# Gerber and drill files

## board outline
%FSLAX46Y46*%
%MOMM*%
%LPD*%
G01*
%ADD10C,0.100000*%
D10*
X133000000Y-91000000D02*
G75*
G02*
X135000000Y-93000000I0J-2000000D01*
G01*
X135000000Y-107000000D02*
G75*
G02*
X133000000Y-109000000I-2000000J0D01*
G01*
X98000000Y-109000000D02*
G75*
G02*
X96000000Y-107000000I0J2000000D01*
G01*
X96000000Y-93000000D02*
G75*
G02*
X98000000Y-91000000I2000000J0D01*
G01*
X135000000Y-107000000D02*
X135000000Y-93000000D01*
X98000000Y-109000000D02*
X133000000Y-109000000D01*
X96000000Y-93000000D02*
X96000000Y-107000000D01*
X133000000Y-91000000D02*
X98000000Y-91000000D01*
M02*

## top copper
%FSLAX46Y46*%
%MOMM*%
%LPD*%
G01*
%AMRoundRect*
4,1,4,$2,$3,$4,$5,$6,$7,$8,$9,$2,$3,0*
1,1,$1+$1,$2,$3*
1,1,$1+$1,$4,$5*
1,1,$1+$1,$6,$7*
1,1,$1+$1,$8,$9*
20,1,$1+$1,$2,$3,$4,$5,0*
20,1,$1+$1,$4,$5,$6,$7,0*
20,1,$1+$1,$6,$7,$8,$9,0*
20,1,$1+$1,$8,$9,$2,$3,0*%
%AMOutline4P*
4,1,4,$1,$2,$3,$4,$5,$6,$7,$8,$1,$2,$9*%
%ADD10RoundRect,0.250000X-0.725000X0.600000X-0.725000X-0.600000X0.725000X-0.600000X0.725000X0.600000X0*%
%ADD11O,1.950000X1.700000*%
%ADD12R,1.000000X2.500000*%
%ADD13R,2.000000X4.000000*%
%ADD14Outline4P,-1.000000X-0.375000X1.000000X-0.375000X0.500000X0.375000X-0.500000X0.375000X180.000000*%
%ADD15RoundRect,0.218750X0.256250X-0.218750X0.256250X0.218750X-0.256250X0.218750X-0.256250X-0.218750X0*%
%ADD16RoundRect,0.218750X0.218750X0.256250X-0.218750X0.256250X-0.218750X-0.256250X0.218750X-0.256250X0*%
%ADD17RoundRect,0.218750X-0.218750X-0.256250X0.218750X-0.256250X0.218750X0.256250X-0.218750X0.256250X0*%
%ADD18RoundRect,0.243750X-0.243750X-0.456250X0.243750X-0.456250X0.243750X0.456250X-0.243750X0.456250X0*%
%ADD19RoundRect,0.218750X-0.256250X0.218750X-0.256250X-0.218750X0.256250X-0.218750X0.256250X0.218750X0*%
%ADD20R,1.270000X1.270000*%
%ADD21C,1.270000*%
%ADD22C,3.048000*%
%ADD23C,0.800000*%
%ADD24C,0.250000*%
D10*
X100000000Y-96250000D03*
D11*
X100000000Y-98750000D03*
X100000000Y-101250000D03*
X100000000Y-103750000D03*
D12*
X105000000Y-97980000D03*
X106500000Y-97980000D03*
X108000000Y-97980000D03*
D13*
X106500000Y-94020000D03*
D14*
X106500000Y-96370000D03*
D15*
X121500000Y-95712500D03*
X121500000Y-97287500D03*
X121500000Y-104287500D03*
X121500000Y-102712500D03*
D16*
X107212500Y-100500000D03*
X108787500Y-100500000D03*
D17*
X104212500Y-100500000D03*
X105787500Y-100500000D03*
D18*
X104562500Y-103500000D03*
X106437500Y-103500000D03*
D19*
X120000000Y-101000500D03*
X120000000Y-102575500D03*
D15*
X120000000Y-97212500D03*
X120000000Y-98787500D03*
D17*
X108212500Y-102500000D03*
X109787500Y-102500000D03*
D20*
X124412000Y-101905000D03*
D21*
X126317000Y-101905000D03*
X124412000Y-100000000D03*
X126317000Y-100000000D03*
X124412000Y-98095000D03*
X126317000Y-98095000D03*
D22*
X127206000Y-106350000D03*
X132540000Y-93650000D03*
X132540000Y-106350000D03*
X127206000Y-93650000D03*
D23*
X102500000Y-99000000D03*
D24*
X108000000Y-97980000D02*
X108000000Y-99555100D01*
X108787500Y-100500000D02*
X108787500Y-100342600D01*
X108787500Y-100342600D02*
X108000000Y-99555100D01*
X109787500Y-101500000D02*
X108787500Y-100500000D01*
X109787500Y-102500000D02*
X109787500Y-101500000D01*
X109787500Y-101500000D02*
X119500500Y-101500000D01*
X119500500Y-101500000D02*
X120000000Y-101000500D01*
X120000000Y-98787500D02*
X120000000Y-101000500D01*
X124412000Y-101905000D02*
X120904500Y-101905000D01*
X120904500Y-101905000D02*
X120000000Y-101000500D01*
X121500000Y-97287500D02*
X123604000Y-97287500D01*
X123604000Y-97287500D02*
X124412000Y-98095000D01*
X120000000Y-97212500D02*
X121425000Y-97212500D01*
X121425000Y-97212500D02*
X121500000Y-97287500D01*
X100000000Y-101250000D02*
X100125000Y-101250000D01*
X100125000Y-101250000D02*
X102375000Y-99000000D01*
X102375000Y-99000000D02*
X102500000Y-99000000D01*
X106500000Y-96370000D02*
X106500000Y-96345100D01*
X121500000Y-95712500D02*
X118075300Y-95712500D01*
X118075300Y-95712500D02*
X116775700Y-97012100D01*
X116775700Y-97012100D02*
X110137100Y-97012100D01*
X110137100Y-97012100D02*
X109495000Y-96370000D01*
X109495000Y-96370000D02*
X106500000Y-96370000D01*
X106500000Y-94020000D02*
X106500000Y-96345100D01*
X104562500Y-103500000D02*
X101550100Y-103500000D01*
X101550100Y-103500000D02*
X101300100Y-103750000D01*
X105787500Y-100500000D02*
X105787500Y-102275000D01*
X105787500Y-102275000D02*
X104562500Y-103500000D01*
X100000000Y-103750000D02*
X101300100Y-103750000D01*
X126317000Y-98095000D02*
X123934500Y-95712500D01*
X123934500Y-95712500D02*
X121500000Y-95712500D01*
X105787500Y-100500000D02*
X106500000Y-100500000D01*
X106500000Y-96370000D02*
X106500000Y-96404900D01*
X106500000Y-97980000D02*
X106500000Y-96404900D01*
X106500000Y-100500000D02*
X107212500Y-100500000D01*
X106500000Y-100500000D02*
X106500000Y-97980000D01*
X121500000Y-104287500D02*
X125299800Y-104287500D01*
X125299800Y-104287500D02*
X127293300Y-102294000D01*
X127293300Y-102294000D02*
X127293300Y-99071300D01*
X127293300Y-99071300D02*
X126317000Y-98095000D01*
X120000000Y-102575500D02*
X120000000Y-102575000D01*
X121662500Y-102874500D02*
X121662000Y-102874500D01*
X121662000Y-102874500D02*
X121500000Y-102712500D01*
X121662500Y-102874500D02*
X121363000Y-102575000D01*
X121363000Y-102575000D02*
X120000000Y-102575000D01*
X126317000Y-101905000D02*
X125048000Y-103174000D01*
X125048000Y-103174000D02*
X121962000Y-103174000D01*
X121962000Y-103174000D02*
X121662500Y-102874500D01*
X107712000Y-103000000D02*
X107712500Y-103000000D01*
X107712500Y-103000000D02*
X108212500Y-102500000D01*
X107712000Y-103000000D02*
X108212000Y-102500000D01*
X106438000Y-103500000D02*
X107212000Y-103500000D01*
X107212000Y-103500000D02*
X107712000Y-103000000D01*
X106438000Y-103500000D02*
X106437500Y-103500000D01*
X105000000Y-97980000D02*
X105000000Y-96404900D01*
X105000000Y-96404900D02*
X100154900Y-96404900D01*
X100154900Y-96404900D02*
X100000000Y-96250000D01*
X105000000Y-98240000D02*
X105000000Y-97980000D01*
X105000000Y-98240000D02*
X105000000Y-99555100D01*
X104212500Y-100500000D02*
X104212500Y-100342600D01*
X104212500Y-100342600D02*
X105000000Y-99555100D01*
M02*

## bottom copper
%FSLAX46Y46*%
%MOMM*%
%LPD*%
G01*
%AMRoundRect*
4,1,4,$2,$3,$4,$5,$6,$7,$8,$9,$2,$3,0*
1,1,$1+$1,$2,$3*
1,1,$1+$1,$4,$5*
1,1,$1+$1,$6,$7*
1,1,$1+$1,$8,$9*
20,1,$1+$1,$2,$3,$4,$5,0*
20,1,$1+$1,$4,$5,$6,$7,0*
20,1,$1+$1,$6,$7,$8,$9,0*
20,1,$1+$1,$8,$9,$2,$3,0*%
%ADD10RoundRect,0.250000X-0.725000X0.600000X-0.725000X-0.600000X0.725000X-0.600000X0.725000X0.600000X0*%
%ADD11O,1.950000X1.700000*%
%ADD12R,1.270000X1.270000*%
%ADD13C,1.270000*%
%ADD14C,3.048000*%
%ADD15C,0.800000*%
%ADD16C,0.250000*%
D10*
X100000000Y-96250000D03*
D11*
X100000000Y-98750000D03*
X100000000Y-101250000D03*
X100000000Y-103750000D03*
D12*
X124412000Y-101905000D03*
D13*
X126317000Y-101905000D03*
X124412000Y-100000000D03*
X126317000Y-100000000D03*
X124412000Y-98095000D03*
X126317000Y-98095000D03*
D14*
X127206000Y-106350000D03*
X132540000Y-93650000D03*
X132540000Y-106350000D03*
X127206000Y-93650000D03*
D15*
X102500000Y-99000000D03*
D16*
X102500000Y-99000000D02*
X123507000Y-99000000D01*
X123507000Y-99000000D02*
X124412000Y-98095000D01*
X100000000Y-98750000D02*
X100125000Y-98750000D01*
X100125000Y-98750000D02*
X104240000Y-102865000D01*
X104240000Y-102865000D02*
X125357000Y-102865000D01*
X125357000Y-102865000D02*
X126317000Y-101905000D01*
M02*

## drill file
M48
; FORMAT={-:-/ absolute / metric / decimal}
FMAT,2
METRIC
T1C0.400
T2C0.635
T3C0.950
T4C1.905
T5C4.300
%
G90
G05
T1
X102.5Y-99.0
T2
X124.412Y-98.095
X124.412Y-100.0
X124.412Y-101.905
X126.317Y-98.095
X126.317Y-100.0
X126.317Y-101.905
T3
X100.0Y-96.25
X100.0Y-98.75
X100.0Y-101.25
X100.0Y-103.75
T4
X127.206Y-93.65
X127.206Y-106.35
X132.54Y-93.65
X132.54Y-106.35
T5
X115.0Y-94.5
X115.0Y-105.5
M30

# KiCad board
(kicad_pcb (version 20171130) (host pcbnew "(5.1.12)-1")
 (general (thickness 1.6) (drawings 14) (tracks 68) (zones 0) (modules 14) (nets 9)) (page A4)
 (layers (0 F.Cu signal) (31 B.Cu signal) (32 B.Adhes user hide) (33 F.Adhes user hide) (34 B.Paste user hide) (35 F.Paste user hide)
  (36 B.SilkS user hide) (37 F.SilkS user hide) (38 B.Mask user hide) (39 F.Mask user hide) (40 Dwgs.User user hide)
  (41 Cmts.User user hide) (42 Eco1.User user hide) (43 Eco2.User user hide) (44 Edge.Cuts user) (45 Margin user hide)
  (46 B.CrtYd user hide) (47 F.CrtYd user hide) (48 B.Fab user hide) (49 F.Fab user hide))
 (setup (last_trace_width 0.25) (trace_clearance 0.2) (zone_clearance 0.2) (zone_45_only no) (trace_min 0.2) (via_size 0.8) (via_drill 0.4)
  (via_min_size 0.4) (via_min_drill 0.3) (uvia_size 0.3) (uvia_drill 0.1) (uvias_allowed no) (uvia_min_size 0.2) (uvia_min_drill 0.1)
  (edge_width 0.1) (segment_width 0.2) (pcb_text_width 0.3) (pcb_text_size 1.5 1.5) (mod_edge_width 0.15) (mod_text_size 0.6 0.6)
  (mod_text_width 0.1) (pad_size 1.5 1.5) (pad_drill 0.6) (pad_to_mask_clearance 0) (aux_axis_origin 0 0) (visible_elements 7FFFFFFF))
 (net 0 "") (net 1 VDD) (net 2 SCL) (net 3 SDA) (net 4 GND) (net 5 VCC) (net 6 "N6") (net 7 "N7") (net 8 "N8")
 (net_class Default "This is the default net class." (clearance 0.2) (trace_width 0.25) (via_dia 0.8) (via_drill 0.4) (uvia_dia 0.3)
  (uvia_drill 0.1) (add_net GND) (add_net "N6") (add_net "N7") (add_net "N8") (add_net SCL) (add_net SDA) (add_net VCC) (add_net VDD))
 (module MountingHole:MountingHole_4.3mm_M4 (layer F.Cu) (at 115 105.5)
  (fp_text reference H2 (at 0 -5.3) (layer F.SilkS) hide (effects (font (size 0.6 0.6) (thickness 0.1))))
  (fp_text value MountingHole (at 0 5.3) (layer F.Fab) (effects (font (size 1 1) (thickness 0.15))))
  (pad 1 np_thru_hole circle (at 0 0) (size 4.3 4.3) (drill 4.3) (layers *.Cu *.Mask)))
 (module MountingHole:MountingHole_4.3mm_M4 (layer F.Cu) (at 115 94.5)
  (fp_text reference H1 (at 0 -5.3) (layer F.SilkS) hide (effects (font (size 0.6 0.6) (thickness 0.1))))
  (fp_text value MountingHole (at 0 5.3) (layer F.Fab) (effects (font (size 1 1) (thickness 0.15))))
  (pad 1 np_thru_hole circle (at 0 0) (size 4.3 4.3) (drill 4.3) (layers *.Cu *.Mask)))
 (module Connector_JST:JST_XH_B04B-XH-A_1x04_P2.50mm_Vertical (layer F.Cu) (at 100 96.25 270)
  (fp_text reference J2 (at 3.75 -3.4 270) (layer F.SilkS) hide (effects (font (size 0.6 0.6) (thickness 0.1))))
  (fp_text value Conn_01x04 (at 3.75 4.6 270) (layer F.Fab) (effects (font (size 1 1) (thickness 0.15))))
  (pad 1 thru_hole roundrect (at 0 0 270) (size 1.7 1.95) (drill 0.95) (layers *.Cu *.Mask) (roundrect_rratio 0.147059) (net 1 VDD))
  (pad 2 thru_hole oval (at 2.5 0 270) (size 1.7 1.95) (drill 0.95) (layers *.Cu *.Mask) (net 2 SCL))
  (pad 3 thru_hole oval (at 5 0 270) (size 1.7 1.95) (drill 0.95) (layers *.Cu *.Mask) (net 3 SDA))
  (pad 4 thru_hole oval (at 7.5 0 270) (size 1.7 1.95) (drill 0.95) (layers *.Cu *.Mask) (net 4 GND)))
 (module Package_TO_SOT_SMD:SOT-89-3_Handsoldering (layer F.Cu) (at 106.5 96 90)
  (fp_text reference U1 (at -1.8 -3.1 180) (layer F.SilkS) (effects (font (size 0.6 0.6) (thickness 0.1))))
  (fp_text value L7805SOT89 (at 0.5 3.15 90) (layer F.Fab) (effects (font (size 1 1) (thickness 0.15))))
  (pad 1 smd rect (at -1.98 -1.5) (size 1 2.5) (layers F.Cu F.Paste F.Mask) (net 1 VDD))
  (pad 2 smd rect (at -1.98 0) (size 1 2.5) (layers F.Cu F.Paste F.Mask) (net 4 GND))
  (pad 3 smd rect (at -1.98 1.5) (size 1 2.5) (layers F.Cu F.Paste F.Mask) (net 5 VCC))
  (pad 2 smd rect (at 1.98 0) (size 2 4) (layers F.Cu F.Paste F.Mask) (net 4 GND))
  (pad 2 smd trapezoid (at -0.37 0 180) (size 1.5 0.75) (rect_delta 0 0.5) (layers F.Cu F.Paste F.Mask) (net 4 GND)))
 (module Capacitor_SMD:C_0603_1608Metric (layer F.Cu) (at 121.5 96.5 90)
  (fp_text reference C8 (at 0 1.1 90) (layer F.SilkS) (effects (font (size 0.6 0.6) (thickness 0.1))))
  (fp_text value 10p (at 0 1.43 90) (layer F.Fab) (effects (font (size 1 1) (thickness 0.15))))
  (pad 2 smd roundrect (at 0.7875 0 90) (size 0.875 0.95) (layers F.Cu F.Paste F.Mask) (roundrect_rratio 0.25) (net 4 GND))
  (pad 1 smd roundrect (at -0.7875 0 90) (size 0.875 0.95) (layers F.Cu F.Paste F.Mask) (roundrect_rratio 0.25) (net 3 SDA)))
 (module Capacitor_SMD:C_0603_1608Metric (layer F.Cu) (at 121.5 103.5 90)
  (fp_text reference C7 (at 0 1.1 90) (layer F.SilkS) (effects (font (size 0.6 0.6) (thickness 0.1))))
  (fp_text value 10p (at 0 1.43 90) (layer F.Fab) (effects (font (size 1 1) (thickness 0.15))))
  (pad 1 smd roundrect (at -0.7875 0 90) (size 0.875 0.95) (layers F.Cu F.Paste F.Mask) (roundrect_rratio 0.25) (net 4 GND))
  (pad 2 smd roundrect (at 0.7875 0 90) (size 0.875 0.95) (layers F.Cu F.Paste F.Mask) (roundrect_rratio 0.25) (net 2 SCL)))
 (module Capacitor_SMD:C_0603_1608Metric (layer F.Cu) (at 108 100.5 180)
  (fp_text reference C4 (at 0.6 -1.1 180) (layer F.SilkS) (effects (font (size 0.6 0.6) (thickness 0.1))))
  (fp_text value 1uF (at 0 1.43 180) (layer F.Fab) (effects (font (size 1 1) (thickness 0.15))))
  (pad 2 smd roundrect (at 0.7875 0 180) (size 0.875 0.95) (layers F.Cu F.Paste F.Mask) (roundrect_rratio 0.25) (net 4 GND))
  (pad 1 smd roundrect (at -0.7875 0 180) (size 0.875 0.95) (layers F.Cu F.Paste F.Mask) (roundrect_rratio 0.25) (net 5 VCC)))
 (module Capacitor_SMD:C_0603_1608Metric (layer F.Cu) (at 105 100.5)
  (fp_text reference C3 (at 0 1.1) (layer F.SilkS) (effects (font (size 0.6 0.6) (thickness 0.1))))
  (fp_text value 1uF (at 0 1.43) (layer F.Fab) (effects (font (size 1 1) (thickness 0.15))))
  (pad 1 smd roundrect (at -0.7875 0) (size 0.875 0.95) (layers F.Cu F.Paste F.Mask) (roundrect_rratio 0.25) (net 1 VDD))
  (pad 2 smd roundrect (at 0.7875 0) (size 0.875 0.95) (layers F.Cu F.Paste F.Mask) (roundrect_rratio 0.25) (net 4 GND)))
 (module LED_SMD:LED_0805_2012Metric (layer F.Cu) (at 105.5 103.5)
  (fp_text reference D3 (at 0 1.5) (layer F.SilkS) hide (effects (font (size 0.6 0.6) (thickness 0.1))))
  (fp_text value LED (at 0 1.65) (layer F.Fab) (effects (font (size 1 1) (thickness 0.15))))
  (pad 1 smd roundrect (at -0.9375 0) (size 0.975 1.4) (layers F.Cu F.Paste F.Mask) (roundrect_rratio 0.25) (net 4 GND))
  (pad 2 smd roundrect (at 0.9375 0) (size 0.975 1.4) (layers F.Cu F.Paste F.Mask) (roundrect_rratio 0.25) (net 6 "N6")))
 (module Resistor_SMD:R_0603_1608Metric (layer F.Cu) (at 120 101.788 270)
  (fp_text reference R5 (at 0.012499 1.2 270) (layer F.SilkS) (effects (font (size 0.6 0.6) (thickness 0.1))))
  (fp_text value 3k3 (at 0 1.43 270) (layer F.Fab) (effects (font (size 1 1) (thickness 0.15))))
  (pad 1 smd roundrect (at -0.7875 0 270) (size 0.875 0.95) (layers F.Cu F.Paste F.Mask) (roundrect_rratio 0.25) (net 5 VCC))
  (pad 2 smd roundrect (at 0.7875 0 270) (size 0.875 0.95) (layers F.Cu F.Paste F.Mask) (roundrect_rratio 0.25) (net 2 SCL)))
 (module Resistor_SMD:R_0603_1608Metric (layer F.Cu) (at 120 98 90)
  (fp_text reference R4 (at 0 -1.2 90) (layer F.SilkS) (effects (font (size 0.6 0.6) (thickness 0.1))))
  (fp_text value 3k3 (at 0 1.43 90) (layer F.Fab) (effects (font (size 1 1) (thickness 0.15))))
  (pad 2 smd roundrect (at 0.7875 0 90) (size 0.875 0.95) (layers F.Cu F.Paste F.Mask) (roundrect_rratio 0.25) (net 3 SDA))
  (pad 1 smd roundrect (at -0.7875 0 90) (size 0.875 0.95) (layers F.Cu F.Paste F.Mask) (roundrect_rratio 0.25) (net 5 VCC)))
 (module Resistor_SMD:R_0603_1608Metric (layer F.Cu) (at 109 102.5)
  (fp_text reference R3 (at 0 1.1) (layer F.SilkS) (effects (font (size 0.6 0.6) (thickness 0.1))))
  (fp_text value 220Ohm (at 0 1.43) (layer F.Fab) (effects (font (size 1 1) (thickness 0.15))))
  (pad 1 smd roundrect (at -0.7875 0) (size 0.875 0.95) (layers F.Cu F.Paste F.Mask) (roundrect_rratio 0.25) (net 6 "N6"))
  (pad 2 smd roundrect (at 0.7875 0) (size 0.875 0.95) (layers F.Cu F.Paste F.Mask) (roundrect_rratio 0.25) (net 5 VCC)))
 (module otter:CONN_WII (layer F.Cu) (at 130 100 270)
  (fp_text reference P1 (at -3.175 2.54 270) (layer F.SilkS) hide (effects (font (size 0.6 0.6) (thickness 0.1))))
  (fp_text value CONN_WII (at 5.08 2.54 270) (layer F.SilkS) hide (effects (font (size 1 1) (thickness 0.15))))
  (pad 1 thru_hole rect (at 1.905 5.588 270) (size 1.27 1.27) (drill 0.635) (layers *.Cu *.Mask F.SilkS) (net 5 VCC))
  (pad 2 thru_hole circle (at 1.905 3.683 270) (size 1.27 1.27) (drill 0.635) (layers *.Cu *.Mask F.SilkS) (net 2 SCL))
  (pad 3 thru_hole circle (at 0 5.588 270) (size 1.27 1.27) (drill 0.635) (layers *.Cu *.Mask F.SilkS) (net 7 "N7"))
  (pad 4 thru_hole circle (at 0 3.683 270) (size 1.27 1.27) (drill 0.635) (layers *.Cu *.Mask F.SilkS) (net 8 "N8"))
  (pad 5 thru_hole circle (at -1.905 5.588 270) (size 1.27 1.27) (drill 0.635) (layers *.Cu *.Mask F.SilkS) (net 3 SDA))
  (pad 6 thru_hole circle (at -1.905 3.683 270) (size 1.27 1.27) (drill 0.635) (layers *.Cu *.Mask F.SilkS) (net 4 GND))
  (pad "" thru_hole circle (at 6.35 2.794 270) (size 3.048 3.048) (drill 1.905) (layers *.Cu *.Mask F.SilkS))
  (pad "" thru_hole circle (at -6.35 -2.54 270) (size 3.048 3.048) (drill 1.905) (layers *.Cu *.Mask F.SilkS))
  (pad "" thru_hole circle (at 6.35 -2.54 270) (size 3.048 3.048) (drill 1.905) (layers *.Cu *.Mask F.SilkS))
  (pad "" thru_hole circle (at -6.35 2.794 270) (size 3.048 3.048) (drill 1.905) (layers *.Cu *.Mask F.SilkS)))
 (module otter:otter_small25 (layer B.Cu) (at 107 100 180)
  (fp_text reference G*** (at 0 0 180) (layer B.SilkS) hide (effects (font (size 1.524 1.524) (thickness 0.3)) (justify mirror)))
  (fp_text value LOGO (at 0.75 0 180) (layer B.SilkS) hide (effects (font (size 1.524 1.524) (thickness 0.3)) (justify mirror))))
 (gr_arc (start 133 93) (end 135 93) (angle -90) (layer Edge.Cuts) (width 0.1))
 (gr_arc (start 133 107) (end 133 109) (angle -90) (layer Edge.Cuts) (width 0.1))
 (gr_arc (start 98 107) (end 96 107) (angle -90) (layer Edge.Cuts) (width 0.1))
 (gr_arc (start 98 93) (end 98 91) (angle -90) (layer Edge.Cuts) (width 0.1))
 (gr_line (start 135 107) (end 135 93) (layer Edge.Cuts) (width 0.1))
 (gr_line (start 98 109) (end 133 109) (layer Edge.Cuts) (width 0.1))
 (gr_line (start 96 93) (end 96 107) (layer Edge.Cuts) (width 0.1))
 (gr_line (start 133 91) (end 98 91) (layer Edge.Cuts) (width 0.1))
 (segment (start 108 97.98) (end 108 99.5551) (width 0.25) (layer F.Cu) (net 5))
 (segment (start 108.7875 100.5) (end 108.7875 100.3426) (width 0.25) (layer F.Cu) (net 5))
 (segment (start 108.7875 100.3426) (end 108 99.5551) (width 0.25) (layer F.Cu) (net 5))
 (segment (start 109.7875 101.5) (end 108.7875 100.5) (width 0.25) (layer F.Cu) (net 5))
 (segment (start 109.7875 102.5) (end 109.7875 101.5) (width 0.25) (layer F.Cu) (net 5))
 (segment (start 109.7875 101.5) (end 119.5005 101.5) (width 0.25) (layer F.Cu) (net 5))
 (segment (start 119.5005 101.5) (end 120 101.0005) (width 0.25) (layer F.Cu) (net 5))
 (segment (start 120 98.7875) (end 120 101.0005) (width 0.25) (layer F.Cu) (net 5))
 (segment (start 124.412 101.905) (end 120.9045 101.905) (width 0.25) (layer F.Cu) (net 5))
 (segment (start 120.9045 101.905) (end 120 101.0005) (width 0.25) (layer F.Cu) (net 5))
 (segment (start 121.5 97.2875) (end 123.604 97.2875) (width 0.25) (layer F.Cu) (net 3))
 (segment (start 123.604 97.2875) (end 124.412 98.095) (width 0.25) (layer F.Cu) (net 3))
 (segment (start 120 97.2125) (end 121.425 97.2125) (width 0.25) (layer F.Cu) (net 3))
 (segment (start 121.425 97.2125) (end 121.5 97.2875) (width 0.25) (layer F.Cu) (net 3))
 (segment (start 102.5 99) (end 123.507 99) (width 0.25) (layer B.Cu) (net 3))
 (segment (start 123.507 99) (end 124.412 98.095) (width 0.25) (layer B.Cu) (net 3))
 (segment (start 100 101.25) (end 100.125 101.25) (width 0.25) (layer F.Cu) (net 3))
 (segment (start 100.125 101.25) (end 102.375 99) (width 0.25) (layer F.Cu) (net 3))
 (segment (start 102.375 99) (end 102.5 99) (width 0.25) (layer F.Cu) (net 3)) (via (at 102.5 99) (size 0.8) (layers F.Cu B.Cu) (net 3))
 (segment (start 106.5 96.37) (end 106.5 96.3451) (width 0.25) (layer F.Cu) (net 4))
 (segment (start 121.5 95.7125) (end 118.0753 95.7125) (width 0.25) (layer F.Cu) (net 4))
 (segment (start 118.0753 95.7125) (end 116.7757 97.0121) (width 0.25) (layer F.Cu) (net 4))
 (segment (start 116.7757 97.0121) (end 110.1371 97.0121) (width 0.25) (layer F.Cu) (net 4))
 (segment (start 110.1371 97.0121) (end 109.495 96.37) (width 0.25) (layer F.Cu) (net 4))
 (segment (start 109.495 96.37) (end 106.5 96.37) (width 0.25) (layer F.Cu) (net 4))
 (segment (start 106.5 94.02) (end 106.5 96.3451) (width 0.25) (layer F.Cu) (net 4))
 (segment (start 104.5625 103.5) (end 101.5501 103.5) (width 0.25) (layer F.Cu) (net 4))
 (segment (start 101.5501 103.5) (end 101.3001 103.75) (width 0.25) (layer F.Cu) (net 4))
 (segment (start 105.7875 100.5) (end 105.7875 102.275) (width 0.25) (layer F.Cu) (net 4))
 (segment (start 105.7875 102.275) (end 104.5625 103.5) (width 0.25) (layer F.Cu) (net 4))
 (segment (start 100 103.75) (end 101.3001 103.75) (width 0.25) (layer F.Cu) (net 4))
 (segment (start 126.317 98.095) (end 123.9345 95.7125) (width 0.25) (layer F.Cu) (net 4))
 (segment (start 123.9345 95.7125) (end 121.5 95.7125) (width 0.25) (layer F.Cu) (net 4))
 (segment (start 105.7875 100.5) (end 106.5 100.5) (width 0.25) (layer F.Cu) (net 4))
 (segment (start 106.5 96.37) (end 106.5 96.4049) (width 0.25) (layer F.Cu) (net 4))
 (segment (start 106.5 97.98) (end 106.5 96.4049) (width 0.25) (layer F.Cu) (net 4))
 (segment (start 106.5 100.5) (end 107.2125 100.5) (width 0.25) (layer F.Cu) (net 4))
 (segment (start 106.5 100.5) (end 106.5 97.98) (width 0.25) (layer F.Cu) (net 4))
 (segment (start 121.5 104.2875) (end 125.2998 104.2875) (width 0.25) (layer F.Cu) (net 4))
 (segment (start 125.2998 104.2875) (end 127.2933 102.294) (width 0.25) (layer F.Cu) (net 4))
 (segment (start 127.2933 102.294) (end 127.2933 99.0713) (width 0.25) (layer F.Cu) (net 4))
 (segment (start 127.2933 99.0713) (end 126.317 98.095) (width 0.25) (layer F.Cu) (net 4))
 (segment (start 120 102.5755) (end 120 102.575) (width 0.25) (layer F.Cu) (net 2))
 (segment (start 121.6625 102.8745) (end 121.662 102.8745) (width 0.25) (layer F.Cu) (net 2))
 (segment (start 121.662 102.8745) (end 121.5 102.7125) (width 0.25) (layer F.Cu) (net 2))
 (segment (start 121.6625 102.8745) (end 121.363 102.575) (width 0.25) (layer F.Cu) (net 2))
 (segment (start 121.363 102.575) (end 120 102.575) (width 0.25) (layer F.Cu) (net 2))
 (segment (start 126.317 101.905) (end 125.048 103.174) (width 0.25) (layer F.Cu) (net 2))
 (segment (start 125.048 103.174) (end 121.962 103.174) (width 0.25) (layer F.Cu) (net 2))
 (segment (start 121.962 103.174) (end 121.6625 102.8745) (width 0.25) (layer F.Cu) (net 2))
 (segment (start 100 98.75) (end 100.125 98.75) (width 0.25) (layer B.Cu) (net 2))
 (segment (start 100.125 98.75) (end 104.24 102.865) (width 0.25) (layer B.Cu) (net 2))
 (segment (start 104.24 102.865) (end 125.357 102.865) (width 0.25) (layer B.Cu) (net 2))
 (segment (start 125.357 102.865) (end 126.317 101.905) (width 0.25) (layer B.Cu) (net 2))
 (segment (start 107.712 103) (end 107.7125 103) (width 0.25) (layer F.Cu) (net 6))
 (segment (start 107.7125 103) (end 108.2125 102.5) (width 0.25) (layer F.Cu) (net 6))
 (segment (start 107.712 103) (end 108.212 102.5) (width 0.25) (layer F.Cu) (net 6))
 (segment (start 106.438 103.5) (end 107.212 103.5) (width 0.25) (layer F.Cu) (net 6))
 (segment (start 107.212 103.5) (end 107.712 103) (width 0.25) (layer F.Cu) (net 6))
 (segment (start 106.438 103.5) (end 106.4375 103.5) (width 0.25) (layer F.Cu) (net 6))
 (segment (start 105 97.98) (end 105 96.4049) (width 0.25) (layer F.Cu) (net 1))
 (segment (start 105 96.4049) (end 100.1549 96.4049) (width 0.25) (layer F.Cu) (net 1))
 (segment (start 100.1549 96.4049) (end 100 96.25) (width 0.25) (layer F.Cu) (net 1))
 (segment (start 105 98.24) (end 105 97.98) (width 0.25) (layer F.Cu) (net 1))
 (segment (start 105 98.24) (end 105 99.5551) (width 0.25) (layer F.Cu) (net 1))
 (segment (start 104.2125 100.5) (end 104.2125 100.3426) (width 0.25) (layer F.Cu) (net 1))
 (segment (start 104.2125 100.3426) (end 105 99.5551) (width 0.25) (layer F.Cu) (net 1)))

